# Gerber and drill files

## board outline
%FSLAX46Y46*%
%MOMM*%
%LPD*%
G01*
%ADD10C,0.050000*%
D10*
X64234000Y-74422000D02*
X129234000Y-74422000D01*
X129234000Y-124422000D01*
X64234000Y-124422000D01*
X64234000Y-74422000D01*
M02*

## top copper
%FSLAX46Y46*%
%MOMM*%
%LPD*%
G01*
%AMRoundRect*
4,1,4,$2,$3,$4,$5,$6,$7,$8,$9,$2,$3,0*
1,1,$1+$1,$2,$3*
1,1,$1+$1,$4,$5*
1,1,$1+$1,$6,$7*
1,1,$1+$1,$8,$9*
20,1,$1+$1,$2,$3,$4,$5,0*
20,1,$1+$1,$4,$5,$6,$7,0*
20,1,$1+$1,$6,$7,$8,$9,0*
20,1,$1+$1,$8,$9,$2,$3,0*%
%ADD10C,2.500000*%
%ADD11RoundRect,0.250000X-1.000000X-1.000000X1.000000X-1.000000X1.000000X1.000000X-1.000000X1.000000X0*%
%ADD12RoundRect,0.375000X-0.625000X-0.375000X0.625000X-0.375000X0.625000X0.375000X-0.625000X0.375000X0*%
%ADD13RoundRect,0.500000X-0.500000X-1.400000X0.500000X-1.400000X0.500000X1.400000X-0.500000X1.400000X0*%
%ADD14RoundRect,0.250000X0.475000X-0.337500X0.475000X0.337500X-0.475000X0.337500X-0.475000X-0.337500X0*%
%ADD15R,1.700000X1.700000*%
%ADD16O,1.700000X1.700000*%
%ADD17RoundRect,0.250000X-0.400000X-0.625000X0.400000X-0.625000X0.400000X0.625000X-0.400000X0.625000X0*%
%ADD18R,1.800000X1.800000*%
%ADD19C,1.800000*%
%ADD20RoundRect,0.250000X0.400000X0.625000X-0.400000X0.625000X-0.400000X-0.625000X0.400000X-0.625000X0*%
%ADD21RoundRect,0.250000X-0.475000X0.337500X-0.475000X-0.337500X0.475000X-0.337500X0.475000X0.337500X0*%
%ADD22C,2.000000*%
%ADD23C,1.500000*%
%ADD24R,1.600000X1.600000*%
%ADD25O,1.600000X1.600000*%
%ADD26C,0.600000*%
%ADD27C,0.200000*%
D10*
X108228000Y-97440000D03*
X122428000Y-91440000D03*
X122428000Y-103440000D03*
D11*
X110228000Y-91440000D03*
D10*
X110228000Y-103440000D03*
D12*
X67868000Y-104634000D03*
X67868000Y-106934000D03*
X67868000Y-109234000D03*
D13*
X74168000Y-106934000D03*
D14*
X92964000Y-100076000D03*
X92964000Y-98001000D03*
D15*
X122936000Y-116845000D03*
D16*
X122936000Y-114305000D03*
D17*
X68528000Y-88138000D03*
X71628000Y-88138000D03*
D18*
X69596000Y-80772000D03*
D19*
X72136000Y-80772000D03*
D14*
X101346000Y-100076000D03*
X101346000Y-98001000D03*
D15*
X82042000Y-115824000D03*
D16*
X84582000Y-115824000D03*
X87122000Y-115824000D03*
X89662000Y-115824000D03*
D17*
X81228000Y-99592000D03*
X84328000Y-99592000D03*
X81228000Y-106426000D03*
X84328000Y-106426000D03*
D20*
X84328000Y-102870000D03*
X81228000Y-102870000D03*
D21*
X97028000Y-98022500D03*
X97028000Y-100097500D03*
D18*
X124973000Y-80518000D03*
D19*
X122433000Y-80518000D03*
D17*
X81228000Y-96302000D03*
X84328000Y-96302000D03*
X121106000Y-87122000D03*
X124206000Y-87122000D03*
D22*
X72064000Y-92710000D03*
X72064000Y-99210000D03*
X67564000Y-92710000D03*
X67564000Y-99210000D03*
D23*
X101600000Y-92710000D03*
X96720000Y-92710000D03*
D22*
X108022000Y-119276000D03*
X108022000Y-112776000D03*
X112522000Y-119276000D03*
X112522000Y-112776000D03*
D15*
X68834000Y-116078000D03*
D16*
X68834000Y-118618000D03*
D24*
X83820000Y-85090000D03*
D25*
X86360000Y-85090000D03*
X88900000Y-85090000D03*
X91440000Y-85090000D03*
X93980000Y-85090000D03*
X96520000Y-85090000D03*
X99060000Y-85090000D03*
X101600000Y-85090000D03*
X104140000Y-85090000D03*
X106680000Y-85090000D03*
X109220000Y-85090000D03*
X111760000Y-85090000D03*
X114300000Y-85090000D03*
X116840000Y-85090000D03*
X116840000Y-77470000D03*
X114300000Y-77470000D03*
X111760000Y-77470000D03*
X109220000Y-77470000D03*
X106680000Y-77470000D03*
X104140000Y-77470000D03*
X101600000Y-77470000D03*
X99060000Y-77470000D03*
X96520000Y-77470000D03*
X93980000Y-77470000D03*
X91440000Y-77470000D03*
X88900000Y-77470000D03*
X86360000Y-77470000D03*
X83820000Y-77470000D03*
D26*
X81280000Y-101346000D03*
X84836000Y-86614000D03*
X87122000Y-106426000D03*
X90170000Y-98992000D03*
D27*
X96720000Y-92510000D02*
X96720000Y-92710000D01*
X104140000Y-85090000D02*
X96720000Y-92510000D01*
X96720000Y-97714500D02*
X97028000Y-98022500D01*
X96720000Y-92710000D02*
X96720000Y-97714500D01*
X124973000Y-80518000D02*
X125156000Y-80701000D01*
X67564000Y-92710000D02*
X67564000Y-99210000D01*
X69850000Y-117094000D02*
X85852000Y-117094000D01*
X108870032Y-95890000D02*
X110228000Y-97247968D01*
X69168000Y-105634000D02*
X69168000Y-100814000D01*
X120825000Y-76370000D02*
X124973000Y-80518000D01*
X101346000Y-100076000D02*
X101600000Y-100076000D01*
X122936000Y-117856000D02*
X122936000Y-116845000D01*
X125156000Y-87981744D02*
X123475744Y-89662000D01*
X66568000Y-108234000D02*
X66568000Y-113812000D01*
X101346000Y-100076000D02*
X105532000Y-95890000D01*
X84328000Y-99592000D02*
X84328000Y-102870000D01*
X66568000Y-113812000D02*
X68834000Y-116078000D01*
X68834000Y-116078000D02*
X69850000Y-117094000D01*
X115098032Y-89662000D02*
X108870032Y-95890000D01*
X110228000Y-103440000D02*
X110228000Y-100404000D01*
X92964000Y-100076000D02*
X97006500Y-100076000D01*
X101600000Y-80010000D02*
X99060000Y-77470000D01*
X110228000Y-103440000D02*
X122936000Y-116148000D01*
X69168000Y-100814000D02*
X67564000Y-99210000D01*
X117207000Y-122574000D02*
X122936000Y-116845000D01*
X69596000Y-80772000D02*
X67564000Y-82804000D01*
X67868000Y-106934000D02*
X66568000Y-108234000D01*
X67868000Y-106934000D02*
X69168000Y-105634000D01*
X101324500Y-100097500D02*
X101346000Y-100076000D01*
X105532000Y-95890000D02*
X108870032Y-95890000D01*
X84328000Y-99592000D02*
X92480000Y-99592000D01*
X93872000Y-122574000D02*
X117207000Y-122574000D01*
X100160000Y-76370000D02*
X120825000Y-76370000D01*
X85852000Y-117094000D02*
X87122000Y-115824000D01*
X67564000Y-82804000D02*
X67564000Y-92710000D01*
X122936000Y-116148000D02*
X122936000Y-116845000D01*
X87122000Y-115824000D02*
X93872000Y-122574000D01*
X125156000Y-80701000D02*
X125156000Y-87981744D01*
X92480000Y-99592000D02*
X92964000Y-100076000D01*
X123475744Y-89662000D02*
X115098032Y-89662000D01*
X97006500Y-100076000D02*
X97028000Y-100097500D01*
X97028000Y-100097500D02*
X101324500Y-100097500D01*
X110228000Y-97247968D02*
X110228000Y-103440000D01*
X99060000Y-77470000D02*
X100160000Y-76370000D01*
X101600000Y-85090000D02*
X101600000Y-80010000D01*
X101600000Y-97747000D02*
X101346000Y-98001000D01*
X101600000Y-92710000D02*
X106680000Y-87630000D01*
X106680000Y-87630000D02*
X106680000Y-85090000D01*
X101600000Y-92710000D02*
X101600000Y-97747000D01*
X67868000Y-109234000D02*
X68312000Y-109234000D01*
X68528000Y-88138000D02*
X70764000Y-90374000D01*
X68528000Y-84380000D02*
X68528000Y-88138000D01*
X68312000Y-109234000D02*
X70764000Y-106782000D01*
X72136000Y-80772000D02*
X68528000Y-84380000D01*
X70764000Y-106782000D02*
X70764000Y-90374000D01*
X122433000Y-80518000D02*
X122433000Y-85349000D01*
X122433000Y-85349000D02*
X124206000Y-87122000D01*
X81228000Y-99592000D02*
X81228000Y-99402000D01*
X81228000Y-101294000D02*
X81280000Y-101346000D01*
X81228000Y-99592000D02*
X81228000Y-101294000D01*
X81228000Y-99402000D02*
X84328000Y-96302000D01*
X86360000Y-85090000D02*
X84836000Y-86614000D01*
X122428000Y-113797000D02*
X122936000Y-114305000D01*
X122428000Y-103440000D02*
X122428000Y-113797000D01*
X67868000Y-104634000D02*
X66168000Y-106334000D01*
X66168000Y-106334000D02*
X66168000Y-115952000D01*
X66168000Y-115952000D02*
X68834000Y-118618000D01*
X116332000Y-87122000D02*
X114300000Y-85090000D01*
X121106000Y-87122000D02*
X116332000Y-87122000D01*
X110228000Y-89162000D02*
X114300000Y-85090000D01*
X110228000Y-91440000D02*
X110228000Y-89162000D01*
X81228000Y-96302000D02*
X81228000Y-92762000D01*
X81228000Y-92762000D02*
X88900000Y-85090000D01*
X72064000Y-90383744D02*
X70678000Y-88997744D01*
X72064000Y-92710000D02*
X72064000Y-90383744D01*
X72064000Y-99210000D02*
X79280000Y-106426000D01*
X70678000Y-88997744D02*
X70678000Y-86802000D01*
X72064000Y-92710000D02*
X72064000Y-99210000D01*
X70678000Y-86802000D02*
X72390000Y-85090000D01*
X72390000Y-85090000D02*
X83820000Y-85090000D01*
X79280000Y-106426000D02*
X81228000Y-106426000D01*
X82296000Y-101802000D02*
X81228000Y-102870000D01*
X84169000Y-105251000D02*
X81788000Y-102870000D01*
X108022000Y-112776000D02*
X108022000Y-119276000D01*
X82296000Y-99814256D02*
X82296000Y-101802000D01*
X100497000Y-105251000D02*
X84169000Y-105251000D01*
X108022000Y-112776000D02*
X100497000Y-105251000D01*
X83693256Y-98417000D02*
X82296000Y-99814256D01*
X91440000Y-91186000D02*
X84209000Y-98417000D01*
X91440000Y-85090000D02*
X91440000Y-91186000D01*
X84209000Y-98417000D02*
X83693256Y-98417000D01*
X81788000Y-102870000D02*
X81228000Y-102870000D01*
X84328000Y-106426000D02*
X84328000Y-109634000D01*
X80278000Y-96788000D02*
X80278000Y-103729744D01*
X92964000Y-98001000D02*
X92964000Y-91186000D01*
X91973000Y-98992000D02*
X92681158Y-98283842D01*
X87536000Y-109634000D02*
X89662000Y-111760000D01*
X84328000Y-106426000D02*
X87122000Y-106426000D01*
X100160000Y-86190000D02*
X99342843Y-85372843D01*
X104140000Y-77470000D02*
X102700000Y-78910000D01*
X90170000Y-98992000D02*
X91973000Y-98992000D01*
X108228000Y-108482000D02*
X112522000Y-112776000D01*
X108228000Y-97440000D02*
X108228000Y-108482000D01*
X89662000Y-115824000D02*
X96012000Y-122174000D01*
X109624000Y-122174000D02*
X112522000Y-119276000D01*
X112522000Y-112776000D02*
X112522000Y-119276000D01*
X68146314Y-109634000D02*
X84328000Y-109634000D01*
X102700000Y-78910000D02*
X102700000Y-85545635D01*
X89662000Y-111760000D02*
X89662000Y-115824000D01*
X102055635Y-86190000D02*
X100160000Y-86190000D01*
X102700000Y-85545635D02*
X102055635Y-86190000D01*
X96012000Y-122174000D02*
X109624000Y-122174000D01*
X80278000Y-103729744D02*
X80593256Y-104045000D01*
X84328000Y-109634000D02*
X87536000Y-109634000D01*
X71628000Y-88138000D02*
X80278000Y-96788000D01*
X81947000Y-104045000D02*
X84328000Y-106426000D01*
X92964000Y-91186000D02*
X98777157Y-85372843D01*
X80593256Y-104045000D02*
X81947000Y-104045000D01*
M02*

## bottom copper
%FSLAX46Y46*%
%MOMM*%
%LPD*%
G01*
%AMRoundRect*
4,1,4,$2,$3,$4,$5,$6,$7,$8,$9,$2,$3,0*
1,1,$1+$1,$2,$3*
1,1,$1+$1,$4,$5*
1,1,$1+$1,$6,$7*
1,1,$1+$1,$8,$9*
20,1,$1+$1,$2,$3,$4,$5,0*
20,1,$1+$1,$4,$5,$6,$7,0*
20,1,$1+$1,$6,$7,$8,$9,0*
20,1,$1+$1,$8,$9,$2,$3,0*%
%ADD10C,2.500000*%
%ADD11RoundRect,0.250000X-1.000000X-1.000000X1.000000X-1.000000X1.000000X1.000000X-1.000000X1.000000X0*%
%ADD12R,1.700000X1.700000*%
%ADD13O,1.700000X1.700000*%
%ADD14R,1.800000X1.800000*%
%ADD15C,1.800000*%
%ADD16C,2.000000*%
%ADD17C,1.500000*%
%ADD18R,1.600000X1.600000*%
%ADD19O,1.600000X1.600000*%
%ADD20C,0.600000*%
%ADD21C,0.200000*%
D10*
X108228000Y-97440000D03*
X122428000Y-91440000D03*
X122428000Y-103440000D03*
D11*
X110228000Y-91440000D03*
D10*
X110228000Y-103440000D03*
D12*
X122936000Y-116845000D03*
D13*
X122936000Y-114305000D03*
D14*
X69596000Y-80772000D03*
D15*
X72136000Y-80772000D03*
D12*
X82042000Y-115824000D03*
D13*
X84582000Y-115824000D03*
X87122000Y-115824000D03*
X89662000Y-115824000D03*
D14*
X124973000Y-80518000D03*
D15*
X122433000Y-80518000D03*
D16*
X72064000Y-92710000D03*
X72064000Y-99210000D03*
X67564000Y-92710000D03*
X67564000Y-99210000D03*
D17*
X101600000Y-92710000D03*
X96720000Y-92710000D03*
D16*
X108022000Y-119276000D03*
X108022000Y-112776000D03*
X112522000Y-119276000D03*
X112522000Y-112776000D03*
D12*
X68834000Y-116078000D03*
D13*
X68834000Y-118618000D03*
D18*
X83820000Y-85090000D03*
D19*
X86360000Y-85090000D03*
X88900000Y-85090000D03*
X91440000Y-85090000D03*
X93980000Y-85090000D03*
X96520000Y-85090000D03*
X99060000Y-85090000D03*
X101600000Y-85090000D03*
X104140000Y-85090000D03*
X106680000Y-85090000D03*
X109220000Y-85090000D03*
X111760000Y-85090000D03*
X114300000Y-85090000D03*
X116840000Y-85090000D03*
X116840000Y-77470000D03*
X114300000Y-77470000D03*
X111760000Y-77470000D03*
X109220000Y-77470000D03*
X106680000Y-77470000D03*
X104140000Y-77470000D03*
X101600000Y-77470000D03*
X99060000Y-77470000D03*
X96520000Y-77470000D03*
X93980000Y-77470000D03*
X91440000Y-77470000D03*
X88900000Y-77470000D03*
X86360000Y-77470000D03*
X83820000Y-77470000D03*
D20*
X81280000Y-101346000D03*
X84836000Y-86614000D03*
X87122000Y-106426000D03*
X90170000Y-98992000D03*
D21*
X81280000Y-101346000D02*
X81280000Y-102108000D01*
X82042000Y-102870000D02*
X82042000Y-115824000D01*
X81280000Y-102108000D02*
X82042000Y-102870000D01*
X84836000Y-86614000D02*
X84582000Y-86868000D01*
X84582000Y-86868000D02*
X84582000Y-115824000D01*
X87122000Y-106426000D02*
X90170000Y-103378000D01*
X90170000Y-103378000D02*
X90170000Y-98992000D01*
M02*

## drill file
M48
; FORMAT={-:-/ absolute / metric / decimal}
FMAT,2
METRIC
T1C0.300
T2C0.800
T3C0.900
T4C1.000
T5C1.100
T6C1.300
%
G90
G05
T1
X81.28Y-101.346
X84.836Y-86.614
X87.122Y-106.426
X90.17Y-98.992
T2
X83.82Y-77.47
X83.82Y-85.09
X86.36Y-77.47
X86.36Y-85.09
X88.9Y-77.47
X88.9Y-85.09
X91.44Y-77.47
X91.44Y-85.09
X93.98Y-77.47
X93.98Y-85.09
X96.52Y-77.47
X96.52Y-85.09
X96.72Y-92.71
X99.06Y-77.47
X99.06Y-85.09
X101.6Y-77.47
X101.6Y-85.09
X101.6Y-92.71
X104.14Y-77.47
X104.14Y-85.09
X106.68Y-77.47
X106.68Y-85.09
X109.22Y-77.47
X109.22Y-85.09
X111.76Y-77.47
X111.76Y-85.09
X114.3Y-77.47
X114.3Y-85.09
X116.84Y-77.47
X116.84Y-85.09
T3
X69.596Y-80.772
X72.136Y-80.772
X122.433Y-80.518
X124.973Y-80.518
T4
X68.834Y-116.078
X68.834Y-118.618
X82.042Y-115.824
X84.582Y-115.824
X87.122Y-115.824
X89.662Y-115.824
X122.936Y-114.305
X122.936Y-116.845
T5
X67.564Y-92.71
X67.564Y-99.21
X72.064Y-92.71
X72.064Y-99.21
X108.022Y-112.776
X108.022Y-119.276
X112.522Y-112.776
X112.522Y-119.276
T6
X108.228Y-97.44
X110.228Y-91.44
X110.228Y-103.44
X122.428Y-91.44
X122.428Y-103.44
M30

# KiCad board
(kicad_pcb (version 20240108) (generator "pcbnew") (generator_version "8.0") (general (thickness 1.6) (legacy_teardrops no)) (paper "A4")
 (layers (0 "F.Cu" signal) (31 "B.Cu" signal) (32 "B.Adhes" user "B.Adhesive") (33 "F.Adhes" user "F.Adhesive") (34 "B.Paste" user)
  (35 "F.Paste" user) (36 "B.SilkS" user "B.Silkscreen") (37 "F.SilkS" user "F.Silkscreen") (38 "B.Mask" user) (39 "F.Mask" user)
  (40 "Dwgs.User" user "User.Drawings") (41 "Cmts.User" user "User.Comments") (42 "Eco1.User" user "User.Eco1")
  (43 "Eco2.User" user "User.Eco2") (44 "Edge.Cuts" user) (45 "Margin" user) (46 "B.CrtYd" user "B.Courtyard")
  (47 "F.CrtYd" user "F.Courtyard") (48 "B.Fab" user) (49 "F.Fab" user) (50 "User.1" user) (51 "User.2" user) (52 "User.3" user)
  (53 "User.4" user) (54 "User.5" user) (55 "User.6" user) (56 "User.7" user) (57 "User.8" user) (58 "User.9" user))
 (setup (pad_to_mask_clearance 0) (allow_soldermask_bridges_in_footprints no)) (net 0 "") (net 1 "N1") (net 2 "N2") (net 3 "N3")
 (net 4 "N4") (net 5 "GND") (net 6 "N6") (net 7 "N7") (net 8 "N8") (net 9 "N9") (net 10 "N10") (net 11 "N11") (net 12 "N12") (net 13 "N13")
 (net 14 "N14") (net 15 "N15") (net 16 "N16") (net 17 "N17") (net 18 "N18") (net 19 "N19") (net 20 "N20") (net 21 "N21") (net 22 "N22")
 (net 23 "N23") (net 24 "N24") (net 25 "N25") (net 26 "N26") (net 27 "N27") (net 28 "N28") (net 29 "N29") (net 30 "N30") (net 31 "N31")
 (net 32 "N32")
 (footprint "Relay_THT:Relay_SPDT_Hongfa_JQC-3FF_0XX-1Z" (layer "F.Cu") (at 110.228 91.44)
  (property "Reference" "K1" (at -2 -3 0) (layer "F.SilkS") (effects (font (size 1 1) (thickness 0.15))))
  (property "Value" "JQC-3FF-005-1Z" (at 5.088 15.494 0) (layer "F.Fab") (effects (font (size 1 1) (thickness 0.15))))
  (pad "11" thru_hole circle (at -2 6) (size 2.5 2.5) (drill 1.3) (layers "*.Cu" "*.Mask") (remove_unused_layers no) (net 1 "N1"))
  (pad "12" thru_hole circle (at 12.2 0) (size 2.5 2.5) (drill 1.3) (layers "*.Cu" "*.Mask") (remove_unused_layers no) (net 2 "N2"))
  (pad "14" thru_hole circle (at 12.2 12) (size 2.5 2.5) (drill 1.3) (layers "*.Cu" "*.Mask") (remove_unused_layers no) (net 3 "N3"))
  (pad "A1" thru_hole roundrect (at 0 0) (size 2.5 2.5) (drill 1.3) (layers "*.Cu" "*.Mask") (remove_unused_layers no)
   (roundrect_rratio 0.1) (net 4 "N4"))
  (pad "A2" thru_hole circle (at 0 12) (size 2.5 2.5) (drill 1.3) (layers "*.Cu" "*.Mask") (remove_unused_layers no) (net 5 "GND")))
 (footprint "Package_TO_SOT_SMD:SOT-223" (layer "F.Cu") (at 71.018 106.934)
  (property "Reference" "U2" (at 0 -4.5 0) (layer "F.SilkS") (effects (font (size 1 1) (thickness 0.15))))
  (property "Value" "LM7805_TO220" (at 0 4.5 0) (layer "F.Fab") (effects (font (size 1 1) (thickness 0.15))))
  (pad "1" smd roundrect (at -3.15 -2.3) (size 2 1.5) (layers "F.Cu" "F.Paste" "F.Mask") (roundrect_rratio 0.25) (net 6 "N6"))
  (pad "2" smd roundrect (at -3.15 0) (size 2 1.5) (layers "F.Cu" "F.Paste" "F.Mask") (roundrect_rratio 0.25) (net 5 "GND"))
  (pad "3" smd roundrect (at -3.15 2.3) (size 2 1.5) (layers "F.Cu" "F.Paste" "F.Mask") (roundrect_rratio 0.25) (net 1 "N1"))
  (pad "4" smd roundrect (at 3.15 0) (size 2 3.8) (layers "F.Cu" "F.Paste" "F.Mask") (roundrect_rratio 0.25)))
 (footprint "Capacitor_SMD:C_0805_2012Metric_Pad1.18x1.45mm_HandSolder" (layer "F.Cu") (at 92.964 99.0385 90)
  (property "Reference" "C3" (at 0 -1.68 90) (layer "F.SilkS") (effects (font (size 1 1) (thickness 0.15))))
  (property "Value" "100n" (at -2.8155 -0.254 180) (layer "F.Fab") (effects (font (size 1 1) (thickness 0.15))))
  (pad "1" smd roundrect (at -1.0375 0 90) (size 1.175 1.45) (layers "F.Cu" "F.Paste" "F.Mask") (roundrect_rratio 0.212766) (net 5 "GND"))
  (pad "2" smd roundrect (at 1.0375 0 90) (size 1.175 1.45) (layers "F.Cu" "F.Paste" "F.Mask") (roundrect_rratio 0.212766) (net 1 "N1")))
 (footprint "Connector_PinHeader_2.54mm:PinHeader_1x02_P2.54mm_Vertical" (layer "F.Cu") (at 122.936 116.845 180)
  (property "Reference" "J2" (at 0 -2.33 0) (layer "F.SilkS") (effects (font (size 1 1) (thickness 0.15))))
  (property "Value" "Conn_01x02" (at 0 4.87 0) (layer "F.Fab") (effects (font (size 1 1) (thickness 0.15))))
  (pad "1" thru_hole rect (at 0 0 180) (size 1.7 1.7) (drill 1) (layers "*.Cu" "*.Mask") (remove_unused_layers no) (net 5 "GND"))
  (pad "2" thru_hole oval (at 0 2.54 180) (size 1.7 1.7) (drill 1) (layers "*.Cu" "*.Mask") (remove_unused_layers no) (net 3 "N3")))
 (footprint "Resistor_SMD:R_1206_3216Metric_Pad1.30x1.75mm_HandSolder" (layer "F.Cu") (at 70.078 88.138)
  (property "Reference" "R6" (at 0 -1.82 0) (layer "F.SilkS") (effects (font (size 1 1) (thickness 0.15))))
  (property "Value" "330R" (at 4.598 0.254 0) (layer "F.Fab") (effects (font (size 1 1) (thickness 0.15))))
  (pad "1" smd roundrect (at -1.55 0) (size 1.3 1.75) (layers "F.Cu" "F.Paste" "F.Mask") (roundrect_rratio 0.192308) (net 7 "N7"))
  (pad "2" smd roundrect (at 1.55 0) (size 1.3 1.75) (layers "F.Cu" "F.Paste" "F.Mask") (roundrect_rratio 0.192308) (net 1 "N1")))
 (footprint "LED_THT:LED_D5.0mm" (layer "F.Cu") (at 69.596 80.772)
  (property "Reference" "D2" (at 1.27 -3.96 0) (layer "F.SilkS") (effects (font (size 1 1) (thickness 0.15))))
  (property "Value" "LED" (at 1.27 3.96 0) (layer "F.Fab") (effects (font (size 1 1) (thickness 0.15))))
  (pad "1" thru_hole rect (at 0 0) (size 1.8 1.8) (drill 0.9) (layers "*.Cu" "*.Mask") (remove_unused_layers no) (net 5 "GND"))
  (pad "2" thru_hole circle (at 2.54 0) (size 1.8 1.8) (drill 0.9) (layers "*.Cu" "*.Mask") (remove_unused_layers no) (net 7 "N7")))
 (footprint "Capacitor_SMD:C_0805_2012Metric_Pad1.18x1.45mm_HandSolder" (layer "F.Cu") (at 101.346 99.0385 90)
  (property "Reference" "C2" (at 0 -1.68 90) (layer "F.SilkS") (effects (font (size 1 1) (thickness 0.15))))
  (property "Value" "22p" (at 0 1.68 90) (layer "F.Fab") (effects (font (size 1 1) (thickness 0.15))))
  (pad "1" smd roundrect (at -1.0375 0 90) (size 1.175 1.45) (layers "F.Cu" "F.Paste" "F.Mask") (roundrect_rratio 0.212766) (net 5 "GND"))
  (pad "2" smd roundrect (at 1.0375 0 90) (size 1.175 1.45) (layers "F.Cu" "F.Paste" "F.Mask") (roundrect_rratio 0.212766) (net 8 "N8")))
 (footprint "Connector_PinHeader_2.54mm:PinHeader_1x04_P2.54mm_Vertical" (layer "F.Cu") (at 82.042 115.824 90)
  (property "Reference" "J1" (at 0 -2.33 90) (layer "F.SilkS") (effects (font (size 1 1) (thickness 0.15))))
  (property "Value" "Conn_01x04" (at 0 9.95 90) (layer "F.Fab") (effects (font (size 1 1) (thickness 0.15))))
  (pad "1" thru_hole rect (at 0 0 90) (size 1.7 1.7) (drill 1) (layers "*.Cu" "*.Mask") (remove_unused_layers no) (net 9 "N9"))
  (pad "2" thru_hole oval (at 0 2.54 90) (size 1.7 1.7) (drill 1) (layers "*.Cu" "*.Mask") (remove_unused_layers no) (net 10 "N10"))
  (pad "3" thru_hole oval (at 0 5.08 90) (size 1.7 1.7) (drill 1) (layers "*.Cu" "*.Mask") (remove_unused_layers no) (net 5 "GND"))
  (pad "4" thru_hole oval (at 0 7.62 90) (size 1.7 1.7) (drill 1) (layers "*.Cu" "*.Mask") (remove_unused_layers no) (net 1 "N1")))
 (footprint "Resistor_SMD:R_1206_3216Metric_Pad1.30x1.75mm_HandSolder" (layer "F.Cu") (at 82.778 99.592)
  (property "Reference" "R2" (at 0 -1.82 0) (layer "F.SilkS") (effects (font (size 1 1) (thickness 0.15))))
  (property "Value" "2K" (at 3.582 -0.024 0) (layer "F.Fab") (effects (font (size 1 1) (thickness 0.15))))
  (pad "1" smd roundrect (at -1.55 0) (size 1.3 1.75) (layers "F.Cu" "F.Paste" "F.Mask") (roundrect_rratio 0.192308) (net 9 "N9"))
  (pad "2" smd roundrect (at 1.55 0) (size 1.3 1.75) (layers "F.Cu" "F.Paste" "F.Mask") (roundrect_rratio 0.192308) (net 5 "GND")))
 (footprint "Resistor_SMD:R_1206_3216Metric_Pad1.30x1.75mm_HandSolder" (layer "F.Cu") (at 82.778 106.426)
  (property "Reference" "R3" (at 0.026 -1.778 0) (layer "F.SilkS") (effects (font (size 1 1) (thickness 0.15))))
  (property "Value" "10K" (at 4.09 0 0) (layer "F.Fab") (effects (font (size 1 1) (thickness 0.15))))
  (pad "1" smd roundrect (at -1.55 0) (size 1.3 1.75) (layers "F.Cu" "F.Paste" "F.Mask") (roundrect_rratio 0.192308) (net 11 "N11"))
  (pad "2" smd roundrect (at 1.55 0) (size 1.3 1.75) (layers "F.Cu" "F.Paste" "F.Mask") (roundrect_rratio 0.192308) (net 1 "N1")))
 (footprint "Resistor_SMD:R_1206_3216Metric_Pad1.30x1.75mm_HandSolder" (layer "F.Cu") (at 82.778 102.87 180)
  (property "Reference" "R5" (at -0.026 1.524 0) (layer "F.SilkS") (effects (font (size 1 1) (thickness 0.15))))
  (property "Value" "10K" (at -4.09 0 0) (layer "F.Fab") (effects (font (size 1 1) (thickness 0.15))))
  (pad "1" smd roundrect (at -1.55 0 180) (size 1.3 1.75) (layers "F.Cu" "F.Paste" "F.Mask") (roundrect_rratio 0.192308) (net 5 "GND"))
  (pad "2" smd roundrect (at 1.55 0 180) (size 1.3 1.75) (layers "F.Cu" "F.Paste" "F.Mask") (roundrect_rratio 0.192308) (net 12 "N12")))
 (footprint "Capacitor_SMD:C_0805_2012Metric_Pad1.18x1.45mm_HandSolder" (layer "F.Cu") (at 97.028 99.06 -90)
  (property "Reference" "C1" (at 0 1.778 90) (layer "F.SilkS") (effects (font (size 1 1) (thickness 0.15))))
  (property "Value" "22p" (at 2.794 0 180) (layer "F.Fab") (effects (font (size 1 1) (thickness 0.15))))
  (pad "1" smd roundrect (at -1.0375 0 270) (size 1.175 1.45) (layers "F.Cu" "F.Paste" "F.Mask") (roundrect_rratio 0.212766) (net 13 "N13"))
  (pad "2" smd roundrect (at 1.0375 0 270) (size 1.175 1.45) (layers "F.Cu" "F.Paste" "F.Mask") (roundrect_rratio 0.212766) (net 5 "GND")))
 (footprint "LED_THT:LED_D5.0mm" (layer "F.Cu") (at 124.973 80.518 180)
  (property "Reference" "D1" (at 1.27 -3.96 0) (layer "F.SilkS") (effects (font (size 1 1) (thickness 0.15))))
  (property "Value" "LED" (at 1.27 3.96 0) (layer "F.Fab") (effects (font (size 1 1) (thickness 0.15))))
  (pad "1" thru_hole rect (at 0 0 180) (size 1.8 1.8) (drill 0.9) (layers "*.Cu" "*.Mask") (remove_unused_layers no) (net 5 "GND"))
  (pad "2" thru_hole circle (at 2.54 0 180) (size 1.8 1.8) (drill 0.9) (layers "*.Cu" "*.Mask") (remove_unused_layers no) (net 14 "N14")))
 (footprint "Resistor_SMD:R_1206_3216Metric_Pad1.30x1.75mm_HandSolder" (layer "F.Cu") (at 82.778 96.302)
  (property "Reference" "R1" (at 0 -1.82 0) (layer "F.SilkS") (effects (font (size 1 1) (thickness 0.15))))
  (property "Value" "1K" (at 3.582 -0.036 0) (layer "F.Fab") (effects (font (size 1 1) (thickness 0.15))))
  (pad "1" smd roundrect (at -1.55 0) (size 1.3 1.75) (layers "F.Cu" "F.Paste" "F.Mask") (roundrect_rratio 0.192308) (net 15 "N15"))
  (pad "2" smd roundrect (at 1.55 0) (size 1.3 1.75) (layers "F.Cu" "F.Paste" "F.Mask") (roundrect_rratio 0.192308) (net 9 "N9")))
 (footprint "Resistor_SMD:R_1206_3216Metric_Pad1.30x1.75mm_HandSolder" (layer "F.Cu") (at 122.656 87.122)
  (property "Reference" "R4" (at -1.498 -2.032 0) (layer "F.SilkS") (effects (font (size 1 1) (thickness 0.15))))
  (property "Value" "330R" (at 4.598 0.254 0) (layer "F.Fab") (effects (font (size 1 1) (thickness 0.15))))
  (pad "1" smd roundrect (at -1.55 0) (size 1.3 1.75) (layers "F.Cu" "F.Paste" "F.Mask") (roundrect_rratio 0.192308) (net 4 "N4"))
  (pad "2" smd roundrect (at 1.55 0) (size 1.3 1.75) (layers "F.Cu" "F.Paste" "F.Mask") (roundrect_rratio 0.192308) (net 14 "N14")))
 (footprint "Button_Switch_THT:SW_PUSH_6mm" (layer "F.Cu") (at 72.064 92.71 -90)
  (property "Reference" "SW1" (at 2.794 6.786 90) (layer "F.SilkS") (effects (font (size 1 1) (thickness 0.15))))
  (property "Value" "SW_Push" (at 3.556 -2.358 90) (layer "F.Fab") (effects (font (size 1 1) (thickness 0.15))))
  (pad "1" thru_hole circle (at 0 0) (size 2 2) (drill 1.1) (layers "*.Cu" "*.Mask") (remove_unused_layers no) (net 11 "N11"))
  (pad "1" thru_hole circle (at 6.5 0) (size 2 2) (drill 1.1) (layers "*.Cu" "*.Mask") (remove_unused_layers no) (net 11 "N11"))
  (pad "2" thru_hole circle (at 0 4.5) (size 2 2) (drill 1.1) (layers "*.Cu" "*.Mask") (remove_unused_layers no) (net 5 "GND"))
  (pad "2" thru_hole circle (at 6.5 4.5) (size 2 2) (drill 1.1) (layers "*.Cu" "*.Mask") (remove_unused_layers no) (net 5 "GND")))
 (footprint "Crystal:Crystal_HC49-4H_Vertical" (layer "F.Cu") (at 101.6 92.71 180)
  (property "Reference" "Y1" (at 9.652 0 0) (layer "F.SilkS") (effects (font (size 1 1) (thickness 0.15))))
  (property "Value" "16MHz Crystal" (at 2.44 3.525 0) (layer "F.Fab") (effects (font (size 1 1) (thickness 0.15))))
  (pad "1" thru_hole circle (at 0 0 180) (size 1.5 1.5) (drill 0.8) (layers "*.Cu" "*.Mask") (remove_unused_layers no) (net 8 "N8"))
  (pad "2" thru_hole circle (at 4.88 0 180) (size 1.5 1.5) (drill 0.8) (layers "*.Cu" "*.Mask") (remove_unused_layers no) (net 13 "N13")))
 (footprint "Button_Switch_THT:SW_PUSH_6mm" (layer "F.Cu") (at 108.022 119.276 90)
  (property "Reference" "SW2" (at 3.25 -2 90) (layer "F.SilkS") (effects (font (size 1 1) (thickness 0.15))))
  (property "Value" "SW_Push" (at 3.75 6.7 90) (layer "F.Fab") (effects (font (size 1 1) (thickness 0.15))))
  (pad "1" thru_hole circle (at 0 0 180) (size 2 2) (drill 1.1) (layers "*.Cu" "*.Mask") (remove_unused_layers no) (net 12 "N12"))
  (pad "1" thru_hole circle (at 6.5 0 180) (size 2 2) (drill 1.1) (layers "*.Cu" "*.Mask") (remove_unused_layers no) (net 12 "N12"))
  (pad "2" thru_hole circle (at 0 4.5 180) (size 2 2) (drill 1.1) (layers "*.Cu" "*.Mask") (remove_unused_layers no) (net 1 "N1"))
  (pad "2" thru_hole circle (at 6.5 4.5 180) (size 2 2) (drill 1.1) (layers "*.Cu" "*.Mask") (remove_unused_layers no) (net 1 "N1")))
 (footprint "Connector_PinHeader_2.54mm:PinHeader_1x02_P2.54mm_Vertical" (layer "F.Cu") (at 68.834 116.078)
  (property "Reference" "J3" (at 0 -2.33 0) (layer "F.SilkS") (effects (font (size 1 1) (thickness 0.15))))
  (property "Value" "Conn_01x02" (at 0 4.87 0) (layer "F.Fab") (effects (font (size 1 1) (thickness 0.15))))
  (pad "1" thru_hole rect (at 0 0) (size 1.7 1.7) (drill 1) (layers "*.Cu" "*.Mask") (remove_unused_layers no) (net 5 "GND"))
  (pad "2" thru_hole oval (at 0 2.54) (size 1.7 1.7) (drill 1) (layers "*.Cu" "*.Mask") (remove_unused_layers no) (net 6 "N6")))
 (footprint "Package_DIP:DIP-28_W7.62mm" (layer "F.Cu") (at 83.82 85.09 90)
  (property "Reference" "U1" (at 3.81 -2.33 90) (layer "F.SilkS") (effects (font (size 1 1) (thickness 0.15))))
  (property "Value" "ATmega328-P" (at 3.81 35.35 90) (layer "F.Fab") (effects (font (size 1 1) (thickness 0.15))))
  (pad "1" thru_hole rect (at 0 0 90) (size 1.6 1.6) (drill 0.8) (layers "*.Cu" "*.Mask") (remove_unused_layers no) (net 11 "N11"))
  (pad "2" thru_hole oval (at 0 2.54 90) (size 1.6 1.6) (drill 0.8) (layers "*.Cu" "*.Mask") (remove_unused_layers no) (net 10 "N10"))
  (pad "3" thru_hole oval (at 0 5.08 90) (size 1.6 1.6) (drill 0.8) (layers "*.Cu" "*.Mask") (remove_unused_layers no) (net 15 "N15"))
  (pad "4" thru_hole oval (at 0 7.62 90) (size 1.6 1.6) (drill 0.8) (layers "*.Cu" "*.Mask") (remove_unused_layers no) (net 12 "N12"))
  (pad "5" thru_hole oval (at 0 10.16 90) (size 1.6 1.6) (drill 0.8) (layers "*.Cu" "*.Mask") (remove_unused_layers no) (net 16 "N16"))
  (pad "6" thru_hole oval (at 0 12.7 90) (size 1.6 1.6) (drill 0.8) (layers "*.Cu" "*.Mask") (remove_unused_layers no) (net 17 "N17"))
  (pad "7" thru_hole oval (at 0 15.24 90) (size 1.6 1.6) (drill 0.8) (layers "*.Cu" "*.Mask") (remove_unused_layers no) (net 1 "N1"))
  (pad "8" thru_hole oval (at 0 17.78 90) (size 1.6 1.6) (drill 0.8) (layers "*.Cu" "*.Mask") (remove_unused_layers no) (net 5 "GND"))
  (pad "9" thru_hole oval (at 0 20.32 90) (size 1.6 1.6) (drill 0.8) (layers "*.Cu" "*.Mask") (remove_unused_layers no) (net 13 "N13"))
  (pad "10" thru_hole oval (at 0 22.86 90) (size 1.6 1.6) (drill 0.8) (layers "*.Cu" "*.Mask") (remove_unused_layers no) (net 8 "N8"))
  (pad "11" thru_hole oval (at 0 25.4 90) (size 1.6 1.6) (drill 0.8) (layers "*.Cu" "*.Mask") (remove_unused_layers no) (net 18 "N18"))
  (pad "12" thru_hole oval (at 0 27.94 90) (size 1.6 1.6) (drill 0.8) (layers "*.Cu" "*.Mask") (remove_unused_layers no) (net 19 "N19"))
  (pad "13" thru_hole oval (at 0 30.48 90) (size 1.6 1.6) (drill 0.8) (layers "*.Cu" "*.Mask") (remove_unused_layers no) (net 4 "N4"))
  (pad "14" thru_hole oval (at 0 33.02 90) (size 1.6 1.6) (drill 0.8) (layers "*.Cu" "*.Mask") (remove_unused_layers no) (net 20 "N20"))
  (pad "15" thru_hole oval (at 7.62 33.02 90) (size 1.6 1.6) (drill 0.8) (layers "*.Cu" "*.Mask") (remove_unused_layers no) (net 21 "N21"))
  (pad "16" thru_hole oval (at 7.62 30.48 90) (size 1.6 1.6) (drill 0.8) (layers "*.Cu" "*.Mask") (remove_unused_layers no) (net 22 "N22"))
  (pad "17" thru_hole oval (at 7.62 27.94 90) (size 1.6 1.6) (drill 0.8) (layers "*.Cu" "*.Mask") (remove_unused_layers no) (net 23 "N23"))
  (pad "18" thru_hole oval (at 7.62 25.4 90) (size 1.6 1.6) (drill 0.8) (layers "*.Cu" "*.Mask") (remove_unused_layers no) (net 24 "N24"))
  (pad "19" thru_hole oval (at 7.62 22.86 90) (size 1.6 1.6) (drill 0.8) (layers "*.Cu" "*.Mask") (remove_unused_layers no) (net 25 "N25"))
  (pad "20" thru_hole oval (at 7.62 20.32 90) (size 1.6 1.6) (drill 0.8) (layers "*.Cu" "*.Mask") (remove_unused_layers no) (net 1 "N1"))
  (pad "21" thru_hole oval (at 7.62 17.78 90) (size 1.6 1.6) (drill 0.8) (layers "*.Cu" "*.Mask") (remove_unused_layers no) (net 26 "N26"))
  (pad "22" thru_hole oval (at 7.62 15.24 90) (size 1.6 1.6) (drill 0.8) (layers "*.Cu" "*.Mask") (remove_unused_layers no) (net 5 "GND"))
  (pad "23" thru_hole oval (at 7.62 12.7 90) (size 1.6 1.6) (drill 0.8) (layers "*.Cu" "*.Mask") (remove_unused_layers no) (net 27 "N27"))
  (pad "24" thru_hole oval (at 7.62 10.16 90) (size 1.6 1.6) (drill 0.8) (layers "*.Cu" "*.Mask") (remove_unused_layers no) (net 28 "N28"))
  (pad "25" thru_hole oval (at 7.62 7.62 90) (size 1.6 1.6) (drill 0.8) (layers "*.Cu" "*.Mask") (remove_unused_layers no) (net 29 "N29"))
  (pad "26" thru_hole oval (at 7.62 5.08 90) (size 1.6 1.6) (drill 0.8) (layers "*.Cu" "*.Mask") (remove_unused_layers no) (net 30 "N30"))
  (pad "27" thru_hole oval (at 7.62 2.54 90) (size 1.6 1.6) (drill 0.8) (layers "*.Cu" "*.Mask") (remove_unused_layers no) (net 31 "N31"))
  (pad "28" thru_hole oval (at 7.62 0 90) (size 1.6 1.6) (drill 0.8) (layers "*.Cu" "*.Mask") (remove_unused_layers no) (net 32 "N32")))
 (gr_rect (start 64.234 74.422) (end 129.234 124.422) (stroke (width 0.05) (type default)) (fill none) (layer "Edge.Cuts"))
 (segment (start 96.72 92.51) (end 96.72 92.71) (width 0.2) (layer "F.Cu") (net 13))
 (segment (start 104.14 85.09) (end 96.72 92.51) (width 0.2) (layer "F.Cu") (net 13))
 (segment (start 96.72 97.7145) (end 97.028 98.0225) (width 0.2) (layer "F.Cu") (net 13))
 (segment (start 96.72 92.71) (end 96.72 97.7145) (width 0.2) (layer "F.Cu") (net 13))
 (segment (start 124.973 80.518) (end 125.156 80.701) (width 0.2) (layer "F.Cu") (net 5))
 (segment (start 67.564 92.71) (end 67.564 99.21) (width 0.2) (layer "F.Cu") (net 5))
 (segment (start 69.85 117.094) (end 85.852 117.094) (width 0.2) (layer "F.Cu") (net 5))
 (segment (start 108.870032 95.89) (end 110.228 97.247968) (width 0.2) (layer "F.Cu") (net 5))
 (segment (start 69.168 105.634) (end 69.168 100.814) (width 0.2) (layer "F.Cu") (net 5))
 (segment (start 120.825 76.37) (end 124.973 80.518) (width 0.2) (layer "F.Cu") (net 5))
 (segment (start 101.346 100.076) (end 101.6 100.076) (width 0.2) (layer "F.Cu") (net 5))
 (segment (start 122.936 117.856) (end 122.936 116.845) (width 0.2) (layer "F.Cu") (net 5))
 (segment (start 125.156 87.981744) (end 123.475744 89.662) (width 0.2) (layer "F.Cu") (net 5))
 (segment (start 66.568 108.234) (end 66.568 113.812) (width 0.2) (layer "F.Cu") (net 5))
 (segment (start 101.346 100.076) (end 105.532 95.89) (width 0.2) (layer "F.Cu") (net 5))
 (segment (start 84.328 99.592) (end 84.328 102.87) (width 0.2) (layer "F.Cu") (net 5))
 (segment (start 66.568 113.812) (end 68.834 116.078) (width 0.2) (layer "F.Cu") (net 5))
 (segment (start 68.834 116.078) (end 69.85 117.094) (width 0.2) (layer "F.Cu") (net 5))
 (segment (start 115.098032 89.662) (end 108.870032 95.89) (width 0.2) (layer "F.Cu") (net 5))
 (segment (start 110.228 103.44) (end 110.228 100.404) (width 0.2) (layer "F.Cu") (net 5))
 (segment (start 92.964 100.076) (end 97.0065 100.076) (width 0.2) (layer "F.Cu") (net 5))
 (segment (start 101.6 80.01) (end 99.06 77.47) (width 0.2) (layer "F.Cu") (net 5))
 (segment (start 110.228 103.44) (end 122.936 116.148) (width 0.2) (layer "F.Cu") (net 5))
 (segment (start 69.168 100.814) (end 67.564 99.21) (width 0.2) (layer "F.Cu") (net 5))
 (segment (start 117.207 122.574) (end 122.936 116.845) (width 0.2) (layer "F.Cu") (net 5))
 (segment (start 69.596 80.772) (end 67.564 82.804) (width 0.2) (layer "F.Cu") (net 5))
 (segment (start 67.868 106.934) (end 66.568 108.234) (width 0.2) (layer "F.Cu") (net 5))
 (segment (start 67.868 106.934) (end 69.168 105.634) (width 0.2) (layer "F.Cu") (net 5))
 (segment (start 101.3245 100.0975) (end 101.346 100.076) (width 0.2) (layer "F.Cu") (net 5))
 (segment (start 105.532 95.89) (end 108.870032 95.89) (width 0.2) (layer "F.Cu") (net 5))
 (segment (start 84.328 99.592) (end 92.48 99.592) (width 0.2) (layer "F.Cu") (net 5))
 (segment (start 93.872 122.574) (end 117.207 122.574) (width 0.2) (layer "F.Cu") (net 5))
 (segment (start 100.16 76.37) (end 120.825 76.37) (width 0.2) (layer "F.Cu") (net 5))
 (segment (start 85.852 117.094) (end 87.122 115.824) (width 0.2) (layer "F.Cu") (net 5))
 (segment (start 67.564 82.804) (end 67.564 92.71) (width 0.2) (layer "F.Cu") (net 5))
 (segment (start 122.936 116.148) (end 122.936 116.845) (width 0.2) (layer "F.Cu") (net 5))
 (segment (start 87.122 115.824) (end 93.872 122.574) (width 0.2) (layer "F.Cu") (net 5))
 (segment (start 125.156 80.701) (end 125.156 87.981744) (width 0.2) (layer "F.Cu") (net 5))
 (segment (start 92.48 99.592) (end 92.964 100.076) (width 0.2) (layer "F.Cu") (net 5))
 (segment (start 123.475744 89.662) (end 115.098032 89.662) (width 0.2) (layer "F.Cu") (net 5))
 (segment (start 97.0065 100.076) (end 97.028 100.0975) (width 0.2) (layer "F.Cu") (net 5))
 (segment (start 97.028 100.0975) (end 101.3245 100.0975) (width 0.2) (layer "F.Cu") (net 5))
 (segment (start 110.228 97.247968) (end 110.228 103.44) (width 0.2) (layer "F.Cu") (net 5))
 (segment (start 99.06 77.47) (end 100.16 76.37) (width 0.2) (layer "F.Cu") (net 5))
 (segment (start 101.6 85.09) (end 101.6 80.01) (width 0.2) (layer "F.Cu") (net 5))
 (segment (start 101.6 97.747) (end 101.346 98.001) (width 0.2) (layer "F.Cu") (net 8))
 (segment (start 101.6 92.71) (end 106.68 87.63) (width 0.2) (layer "F.Cu") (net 8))
 (segment (start 106.68 87.63) (end 106.68 85.09) (width 0.2) (layer "F.Cu") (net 8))
 (segment (start 101.6 92.71) (end 101.6 97.747) (width 0.2) (layer "F.Cu") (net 8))
 (segment (start 67.868 109.234) (end 68.312 109.234) (width 0.2) (layer "F.Cu") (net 7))
 (segment (start 68.528 88.138) (end 70.764 90.374) (width 0.2) (layer "F.Cu") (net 7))
 (segment (start 68.528 84.38) (end 68.528 88.138) (width 0.2) (layer "F.Cu") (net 7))
 (segment (start 68.312 109.234) (end 70.764 106.782) (width 0.2) (layer "F.Cu") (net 7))
 (segment (start 72.136 80.772) (end 68.528 84.38) (width 0.2) (layer "F.Cu") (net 7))
 (segment (start 70.764 106.782) (end 70.764 90.374) (width 0.2) (layer "F.Cu") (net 7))
 (segment (start 122.433 80.518) (end 122.433 85.349) (width 0.2) (layer "F.Cu") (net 14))
 (segment (start 122.433 85.349) (end 124.206 87.122) (width 0.2) (layer "F.Cu") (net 14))
 (segment (start 81.228 99.592) (end 81.228 99.402) (width 0.2) (layer "F.Cu") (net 9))
 (segment (start 81.228 101.294) (end 81.28 101.346) (width 0.2) (layer "F.Cu") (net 9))
 (segment (start 81.228 99.592) (end 81.228 101.294) (width 0.2) (layer "F.Cu") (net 9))
 (segment (start 81.228 99.402) (end 84.328 96.302) (width 0.2) (layer "F.Cu") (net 9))
 (via (at 81.28 101.346) (size 0.6) (drill 0.3) (layers "F.Cu" "B.Cu") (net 9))
 (segment (start 81.28 101.346) (end 81.28 102.108) (width 0.2) (layer "B.Cu") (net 9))
 (segment (start 82.042 102.87) (end 82.042 115.824) (width 0.2) (layer "B.Cu") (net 9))
 (segment (start 81.28 102.108) (end 82.042 102.87) (width 0.2) (layer "B.Cu") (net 9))
 (segment (start 86.36 85.09) (end 84.836 86.614) (width 0.2) (layer "F.Cu") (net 10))
 (via (at 84.836 86.614) (size 0.6) (drill 0.3) (layers "F.Cu" "B.Cu") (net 10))
 (segment (start 84.836 86.614) (end 84.582 86.868) (width 0.2) (layer "B.Cu") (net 10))
 (segment (start 84.582 86.868) (end 84.582 115.824) (width 0.2) (layer "B.Cu") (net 10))
 (segment (start 122.428 113.797) (end 122.936 114.305) (width 0.2) (layer "F.Cu") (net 3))
 (segment (start 122.428 103.44) (end 122.428 113.797) (width 0.2) (layer "F.Cu") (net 3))
 (segment (start 67.868 104.634) (end 66.168 106.334) (width 0.2) (layer "F.Cu") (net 6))
 (segment (start 66.168 106.334) (end 66.168 115.952) (width 0.2) (layer "F.Cu") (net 6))
 (segment (start 66.168 115.952) (end 68.834 118.618) (width 0.2) (layer "F.Cu") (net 6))
 (segment (start 116.332 87.122) (end 114.3 85.09) (width 0.2) (layer "F.Cu") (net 4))
 (segment (start 121.106 87.122) (end 116.332 87.122) (width 0.2) (layer "F.Cu") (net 4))
 (segment (start 110.228 89.162) (end 114.3 85.09) (width 0.2) (layer "F.Cu") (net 4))
 (segment (start 110.228 91.44) (end 110.228 89.162) (width 0.2) (layer "F.Cu") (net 4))
 (segment (start 81.228 96.302) (end 81.228 92.762) (width 0.2) (layer "F.Cu") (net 15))
 (segment (start 81.228 92.762) (end 88.9 85.09) (width 0.2) (layer "F.Cu") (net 15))
 (segment (start 72.064 90.383744) (end 70.678 88.997744) (width 0.2) (layer "F.Cu") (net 11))
 (segment (start 72.064 92.71) (end 72.064 90.383744) (width 0.2) (layer "F.Cu") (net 11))
 (segment (start 72.064 99.21) (end 79.28 106.426) (width 0.2) (layer "F.Cu") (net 11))
 (segment (start 70.678 88.997744) (end 70.678 86.802) (width 0.2) (layer "F.Cu") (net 11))
 (segment (start 72.064 92.71) (end 72.064 99.21) (width 0.2) (layer "F.Cu") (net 11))
 (segment (start 70.678 86.802) (end 72.39 85.09) (width 0.2) (layer "F.Cu") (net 11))
 (segment (start 72.39 85.09) (end 83.82 85.09) (width 0.2) (layer "F.Cu") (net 11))
 (segment (start 79.28 106.426) (end 81.228 106.426) (width 0.2) (layer "F.Cu") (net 11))
 (segment (start 82.296 101.802) (end 81.228 102.87) (width 0.2) (layer "F.Cu") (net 12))
 (segment (start 84.169 105.251) (end 81.788 102.87) (width 0.2) (layer "F.Cu") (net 12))
 (segment (start 108.022 112.776) (end 108.022 119.276) (width 0.2) (layer "F.Cu") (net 12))
 (segment (start 82.296 99.814256) (end 82.296 101.802) (width 0.2) (layer "F.Cu") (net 12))
 (segment (start 100.497 105.251) (end 84.169 105.251) (width 0.2) (layer "F.Cu") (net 12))
 (segment (start 108.022 112.776) (end 100.497 105.251) (width 0.2) (layer "F.Cu") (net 12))
 (segment (start 83.693256 98.417) (end 82.296 99.814256) (width 0.2) (layer "F.Cu") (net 12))
 (segment (start 91.44 91.186) (end 84.209 98.417) (width 0.2) (layer "F.Cu") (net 12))
 (segment (start 91.44 85.09) (end 91.44 91.186) (width 0.2) (layer "F.Cu") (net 12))
 (segment (start 84.209 98.417) (end 83.693256 98.417) (width 0.2) (layer "F.Cu") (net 12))
 (segment (start 81.788 102.87) (end 81.228 102.87) (width 0.2) (layer "F.Cu") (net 12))
 (segment (start 84.328 106.426) (end 84.328 109.634) (width 0.2) (layer "F.Cu") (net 1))
 (segment (start 80.278 96.788) (end 80.278 103.729744) (width 0.2) (layer "F.Cu") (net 1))
 (segment (start 92.964 98.001) (end 92.964 91.186) (width 0.2) (layer "F.Cu") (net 1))
 (segment (start 91.973 98.992) (end 92.681158 98.283842) (width 0.2) (layer "F.Cu") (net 1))
 (segment (start 87.536 109.634) (end 89.662 111.76) (width 0.2) (layer "F.Cu") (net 1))
 (segment (start 84.328 106.426) (end 87.122 106.426) (width 0.2) (layer "F.Cu") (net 1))
 (segment (start 100.16 86.19) (end 99.342843 85.372843) (width 0.2) (layer "F.Cu") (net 1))
 (segment (start 104.14 77.47) (end 102.7 78.91) (width 0.2) (layer "F.Cu") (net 1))
 (segment (start 90.17 98.992) (end 91.973 98.992) (width 0.2) (layer "F.Cu") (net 1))
 (segment (start 108.228 108.482) (end 112.522 112.776) (width 0.2) (layer "F.Cu") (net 1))
 (segment (start 108.228 97.44) (end 108.228 108.482) (width 0.2) (layer "F.Cu") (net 1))
 (segment (start 89.662 115.824) (end 96.012 122.174) (width 0.2) (layer "F.Cu") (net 1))
 (segment (start 109.624 122.174) (end 112.522 119.276) (width 0.2) (layer "F.Cu") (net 1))
 (segment (start 112.522 112.776) (end 112.522 119.276) (width 0.2) (layer "F.Cu") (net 1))
 (segment (start 68.146314 109.634) (end 84.328 109.634) (width 0.2) (layer "F.Cu") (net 1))
 (segment (start 102.7 78.91) (end 102.7 85.545635) (width 0.2) (layer "F.Cu") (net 1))
 (segment (start 89.662 111.76) (end 89.662 115.824) (width 0.2) (layer "F.Cu") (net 1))
 (segment (start 102.055635 86.19) (end 100.16 86.19) (width 0.2) (layer "F.Cu") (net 1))
 (segment (start 102.7 85.545635) (end 102.055635 86.19) (width 0.2) (layer "F.Cu") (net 1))
 (segment (start 96.012 122.174) (end 109.624 122.174) (width 0.2) (layer "F.Cu") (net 1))
 (segment (start 80.278 103.729744) (end 80.593256 104.045) (width 0.2) (layer "F.Cu") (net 1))
 (segment (start 84.328 109.634) (end 87.536 109.634) (width 0.2) (layer "F.Cu") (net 1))
 (segment (start 71.628 88.138) (end 80.278 96.788) (width 0.2) (layer "F.Cu") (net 1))
 (segment (start 81.947 104.045) (end 84.328 106.426) (width 0.2) (layer "F.Cu") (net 1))
 (segment (start 92.964 91.186) (end 98.777157 85.372843) (width 0.2) (layer "F.Cu") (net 1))
 (segment (start 80.593256 104.045) (end 81.947 104.045) (width 0.2) (layer "F.Cu") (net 1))
 (via (at 87.122 106.426) (size 0.6) (drill 0.3) (layers "F.Cu" "B.Cu") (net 1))
 (via (at 90.17 98.992) (size 0.6) (drill 0.3) (layers "F.Cu" "B.Cu") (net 1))
 (segment (start 87.122 106.426) (end 90.17 103.378) (width 0.2) (layer "B.Cu") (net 1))
 (segment (start 90.17 103.378) (end 90.17 98.992) (width 0.2) (layer "B.Cu") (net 1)))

